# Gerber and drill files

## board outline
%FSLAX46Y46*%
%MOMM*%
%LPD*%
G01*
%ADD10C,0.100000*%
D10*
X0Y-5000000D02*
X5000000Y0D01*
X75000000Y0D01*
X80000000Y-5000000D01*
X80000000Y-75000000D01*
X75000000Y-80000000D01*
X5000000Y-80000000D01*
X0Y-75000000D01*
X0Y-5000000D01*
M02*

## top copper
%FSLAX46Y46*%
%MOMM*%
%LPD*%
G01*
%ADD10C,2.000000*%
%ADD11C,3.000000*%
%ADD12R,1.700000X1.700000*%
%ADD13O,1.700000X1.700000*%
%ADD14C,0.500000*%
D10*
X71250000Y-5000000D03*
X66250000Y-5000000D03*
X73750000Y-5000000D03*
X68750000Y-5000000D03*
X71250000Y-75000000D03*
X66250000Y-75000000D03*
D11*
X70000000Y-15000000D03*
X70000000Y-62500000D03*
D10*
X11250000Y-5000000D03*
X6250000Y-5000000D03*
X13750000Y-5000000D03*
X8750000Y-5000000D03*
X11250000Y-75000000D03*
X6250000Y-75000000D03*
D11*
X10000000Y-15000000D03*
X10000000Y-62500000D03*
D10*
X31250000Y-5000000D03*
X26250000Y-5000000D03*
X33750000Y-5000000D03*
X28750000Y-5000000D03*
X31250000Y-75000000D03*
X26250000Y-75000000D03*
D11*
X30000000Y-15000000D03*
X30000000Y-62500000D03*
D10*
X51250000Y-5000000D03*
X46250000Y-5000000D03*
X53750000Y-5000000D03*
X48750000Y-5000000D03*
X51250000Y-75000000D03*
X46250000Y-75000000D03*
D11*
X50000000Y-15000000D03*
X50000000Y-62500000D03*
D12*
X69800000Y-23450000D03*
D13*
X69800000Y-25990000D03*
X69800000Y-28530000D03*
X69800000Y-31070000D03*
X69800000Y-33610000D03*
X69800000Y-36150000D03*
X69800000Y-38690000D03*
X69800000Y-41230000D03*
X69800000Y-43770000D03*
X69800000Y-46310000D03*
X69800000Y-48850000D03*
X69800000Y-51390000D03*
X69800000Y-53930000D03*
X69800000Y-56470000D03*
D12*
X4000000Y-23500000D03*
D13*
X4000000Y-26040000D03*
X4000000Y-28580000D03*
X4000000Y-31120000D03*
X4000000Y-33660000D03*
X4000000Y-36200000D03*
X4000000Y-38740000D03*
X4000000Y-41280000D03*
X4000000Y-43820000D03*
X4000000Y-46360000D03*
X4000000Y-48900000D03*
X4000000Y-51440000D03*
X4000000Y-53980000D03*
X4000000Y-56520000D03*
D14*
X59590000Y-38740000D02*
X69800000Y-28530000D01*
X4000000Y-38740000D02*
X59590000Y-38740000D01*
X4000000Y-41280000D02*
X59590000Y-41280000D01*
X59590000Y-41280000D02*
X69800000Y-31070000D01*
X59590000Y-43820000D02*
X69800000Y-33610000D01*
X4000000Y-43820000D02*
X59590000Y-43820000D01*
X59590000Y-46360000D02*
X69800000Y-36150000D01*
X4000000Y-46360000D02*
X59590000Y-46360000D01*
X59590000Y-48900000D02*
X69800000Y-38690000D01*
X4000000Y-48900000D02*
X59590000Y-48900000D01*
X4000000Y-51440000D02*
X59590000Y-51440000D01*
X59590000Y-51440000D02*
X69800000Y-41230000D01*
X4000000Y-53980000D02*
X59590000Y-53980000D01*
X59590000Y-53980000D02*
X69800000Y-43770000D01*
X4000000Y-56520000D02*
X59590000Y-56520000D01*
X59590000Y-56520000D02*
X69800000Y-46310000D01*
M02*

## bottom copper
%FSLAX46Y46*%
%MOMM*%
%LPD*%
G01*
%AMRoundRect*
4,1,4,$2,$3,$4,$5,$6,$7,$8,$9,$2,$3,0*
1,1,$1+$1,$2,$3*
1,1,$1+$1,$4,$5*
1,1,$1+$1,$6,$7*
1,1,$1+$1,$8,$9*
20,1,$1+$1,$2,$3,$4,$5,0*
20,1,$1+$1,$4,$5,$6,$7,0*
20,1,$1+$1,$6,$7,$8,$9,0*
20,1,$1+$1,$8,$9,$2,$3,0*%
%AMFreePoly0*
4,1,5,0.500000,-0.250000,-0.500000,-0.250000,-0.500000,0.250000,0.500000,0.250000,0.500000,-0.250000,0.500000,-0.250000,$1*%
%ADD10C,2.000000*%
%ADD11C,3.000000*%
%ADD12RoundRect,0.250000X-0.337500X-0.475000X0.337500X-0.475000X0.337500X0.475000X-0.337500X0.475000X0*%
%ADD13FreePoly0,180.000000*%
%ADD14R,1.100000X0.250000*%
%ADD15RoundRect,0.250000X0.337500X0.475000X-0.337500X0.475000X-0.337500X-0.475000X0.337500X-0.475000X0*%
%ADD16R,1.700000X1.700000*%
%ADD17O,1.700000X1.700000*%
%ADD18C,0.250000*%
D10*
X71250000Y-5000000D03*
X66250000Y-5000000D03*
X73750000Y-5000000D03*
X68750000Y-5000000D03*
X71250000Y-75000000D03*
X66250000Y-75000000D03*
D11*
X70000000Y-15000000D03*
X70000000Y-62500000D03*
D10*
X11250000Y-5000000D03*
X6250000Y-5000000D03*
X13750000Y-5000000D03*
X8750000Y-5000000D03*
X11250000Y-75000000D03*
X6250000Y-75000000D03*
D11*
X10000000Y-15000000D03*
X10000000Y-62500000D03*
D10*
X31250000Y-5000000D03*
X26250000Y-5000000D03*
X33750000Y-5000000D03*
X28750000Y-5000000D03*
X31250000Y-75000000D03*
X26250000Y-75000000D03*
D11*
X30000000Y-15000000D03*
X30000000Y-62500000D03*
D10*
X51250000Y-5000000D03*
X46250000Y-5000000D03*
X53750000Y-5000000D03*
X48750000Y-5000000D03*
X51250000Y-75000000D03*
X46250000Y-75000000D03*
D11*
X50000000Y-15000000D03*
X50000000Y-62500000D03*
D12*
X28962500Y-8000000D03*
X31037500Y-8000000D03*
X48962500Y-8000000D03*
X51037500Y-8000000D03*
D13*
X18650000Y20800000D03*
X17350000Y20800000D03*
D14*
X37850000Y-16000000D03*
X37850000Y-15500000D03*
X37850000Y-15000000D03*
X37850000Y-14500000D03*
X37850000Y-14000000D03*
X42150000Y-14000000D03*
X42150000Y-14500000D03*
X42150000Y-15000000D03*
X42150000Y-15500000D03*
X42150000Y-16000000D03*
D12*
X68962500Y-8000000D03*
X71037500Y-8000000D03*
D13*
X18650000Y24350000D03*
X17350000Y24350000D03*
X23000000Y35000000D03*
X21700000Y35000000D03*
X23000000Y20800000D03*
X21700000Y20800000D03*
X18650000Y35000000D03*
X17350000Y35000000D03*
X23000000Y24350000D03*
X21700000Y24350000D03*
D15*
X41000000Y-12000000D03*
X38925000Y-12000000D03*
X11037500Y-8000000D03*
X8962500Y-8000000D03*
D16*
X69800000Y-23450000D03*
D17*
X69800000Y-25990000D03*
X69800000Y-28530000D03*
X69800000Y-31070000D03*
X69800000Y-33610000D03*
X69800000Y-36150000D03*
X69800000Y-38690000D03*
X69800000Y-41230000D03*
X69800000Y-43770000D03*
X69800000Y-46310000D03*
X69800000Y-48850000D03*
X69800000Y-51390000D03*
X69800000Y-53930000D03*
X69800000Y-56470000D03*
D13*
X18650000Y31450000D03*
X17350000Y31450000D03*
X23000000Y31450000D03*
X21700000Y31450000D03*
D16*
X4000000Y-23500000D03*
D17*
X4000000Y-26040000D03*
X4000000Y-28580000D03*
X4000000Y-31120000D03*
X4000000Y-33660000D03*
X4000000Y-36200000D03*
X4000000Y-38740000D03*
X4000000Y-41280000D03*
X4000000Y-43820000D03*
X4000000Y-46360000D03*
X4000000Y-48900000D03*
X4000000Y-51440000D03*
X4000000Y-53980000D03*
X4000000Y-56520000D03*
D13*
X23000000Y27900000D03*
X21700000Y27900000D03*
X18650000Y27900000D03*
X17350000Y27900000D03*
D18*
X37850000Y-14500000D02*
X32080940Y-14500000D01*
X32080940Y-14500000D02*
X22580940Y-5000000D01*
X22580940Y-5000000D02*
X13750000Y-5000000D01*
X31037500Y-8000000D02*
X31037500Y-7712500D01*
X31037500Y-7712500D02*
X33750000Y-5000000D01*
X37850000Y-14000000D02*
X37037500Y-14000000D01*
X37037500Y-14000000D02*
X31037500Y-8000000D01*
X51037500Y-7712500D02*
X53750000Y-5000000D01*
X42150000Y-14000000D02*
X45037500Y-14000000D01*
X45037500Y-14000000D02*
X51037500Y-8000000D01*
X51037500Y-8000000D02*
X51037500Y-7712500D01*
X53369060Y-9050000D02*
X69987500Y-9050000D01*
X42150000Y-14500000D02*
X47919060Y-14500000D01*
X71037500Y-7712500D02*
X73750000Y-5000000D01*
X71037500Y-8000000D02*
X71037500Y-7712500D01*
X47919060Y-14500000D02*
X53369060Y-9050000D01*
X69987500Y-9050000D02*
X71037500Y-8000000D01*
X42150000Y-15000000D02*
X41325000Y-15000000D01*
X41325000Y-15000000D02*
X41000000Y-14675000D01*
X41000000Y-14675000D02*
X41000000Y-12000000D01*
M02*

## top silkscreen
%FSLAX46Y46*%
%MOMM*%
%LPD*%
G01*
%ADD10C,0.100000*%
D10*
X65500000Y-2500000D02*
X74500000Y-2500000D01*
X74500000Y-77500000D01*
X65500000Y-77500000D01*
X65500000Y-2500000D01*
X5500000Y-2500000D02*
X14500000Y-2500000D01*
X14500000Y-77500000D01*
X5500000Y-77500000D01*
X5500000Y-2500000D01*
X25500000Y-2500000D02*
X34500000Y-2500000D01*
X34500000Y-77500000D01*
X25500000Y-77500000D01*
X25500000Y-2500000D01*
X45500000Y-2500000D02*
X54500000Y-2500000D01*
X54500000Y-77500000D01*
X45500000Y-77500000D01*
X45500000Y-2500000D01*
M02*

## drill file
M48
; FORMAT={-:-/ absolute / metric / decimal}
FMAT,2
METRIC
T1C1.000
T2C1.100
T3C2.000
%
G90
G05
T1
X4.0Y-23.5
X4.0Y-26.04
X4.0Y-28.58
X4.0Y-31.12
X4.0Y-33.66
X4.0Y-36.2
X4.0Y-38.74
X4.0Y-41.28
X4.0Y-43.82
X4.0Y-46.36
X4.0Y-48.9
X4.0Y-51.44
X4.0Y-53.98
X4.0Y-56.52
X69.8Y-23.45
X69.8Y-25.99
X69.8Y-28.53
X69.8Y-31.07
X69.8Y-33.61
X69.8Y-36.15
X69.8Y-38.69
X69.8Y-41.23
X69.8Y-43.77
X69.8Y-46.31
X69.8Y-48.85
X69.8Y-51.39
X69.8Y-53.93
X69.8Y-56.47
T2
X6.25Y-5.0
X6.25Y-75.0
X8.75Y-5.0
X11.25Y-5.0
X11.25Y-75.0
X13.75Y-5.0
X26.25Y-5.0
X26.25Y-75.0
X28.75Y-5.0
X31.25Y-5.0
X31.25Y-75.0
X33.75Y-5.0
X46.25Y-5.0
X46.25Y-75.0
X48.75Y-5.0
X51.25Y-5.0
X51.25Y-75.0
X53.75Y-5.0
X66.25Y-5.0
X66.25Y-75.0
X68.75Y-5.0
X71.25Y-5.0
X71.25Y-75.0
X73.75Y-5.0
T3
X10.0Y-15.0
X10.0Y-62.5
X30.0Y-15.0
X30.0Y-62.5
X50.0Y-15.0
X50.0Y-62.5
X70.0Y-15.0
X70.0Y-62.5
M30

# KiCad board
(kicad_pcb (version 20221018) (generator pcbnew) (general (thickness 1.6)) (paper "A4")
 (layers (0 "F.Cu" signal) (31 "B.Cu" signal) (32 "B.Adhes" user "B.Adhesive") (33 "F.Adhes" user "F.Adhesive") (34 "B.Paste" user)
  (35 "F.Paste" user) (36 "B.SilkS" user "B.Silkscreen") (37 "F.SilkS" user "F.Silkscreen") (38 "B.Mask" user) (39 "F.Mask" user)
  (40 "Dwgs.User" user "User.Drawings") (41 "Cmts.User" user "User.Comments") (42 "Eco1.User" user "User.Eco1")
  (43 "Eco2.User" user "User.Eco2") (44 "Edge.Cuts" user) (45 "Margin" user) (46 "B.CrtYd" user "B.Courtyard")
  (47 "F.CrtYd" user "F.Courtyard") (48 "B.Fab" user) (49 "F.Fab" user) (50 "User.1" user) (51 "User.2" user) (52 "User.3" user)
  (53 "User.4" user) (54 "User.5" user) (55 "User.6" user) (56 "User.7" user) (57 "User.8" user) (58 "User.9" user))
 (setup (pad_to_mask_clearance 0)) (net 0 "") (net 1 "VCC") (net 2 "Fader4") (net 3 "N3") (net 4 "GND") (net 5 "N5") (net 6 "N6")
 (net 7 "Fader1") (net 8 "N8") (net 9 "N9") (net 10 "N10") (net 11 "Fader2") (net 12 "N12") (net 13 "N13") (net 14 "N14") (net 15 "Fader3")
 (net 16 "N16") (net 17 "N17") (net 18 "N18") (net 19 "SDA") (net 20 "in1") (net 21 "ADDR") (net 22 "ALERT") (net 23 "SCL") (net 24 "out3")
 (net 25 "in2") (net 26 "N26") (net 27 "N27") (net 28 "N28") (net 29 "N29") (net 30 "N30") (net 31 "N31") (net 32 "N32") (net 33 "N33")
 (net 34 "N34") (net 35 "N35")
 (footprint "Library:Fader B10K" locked (layer "F.Cu") (at 70 5 -90)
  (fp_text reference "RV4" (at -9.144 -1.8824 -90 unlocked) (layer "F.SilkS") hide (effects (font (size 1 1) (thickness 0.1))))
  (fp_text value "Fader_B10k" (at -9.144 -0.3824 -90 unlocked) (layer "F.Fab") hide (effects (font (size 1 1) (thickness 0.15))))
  (fp_rect (start -2.5 -4.5) (end 72.5 4.5) (stroke (width 0.1) (type default)) (fill none) (layer "F.SilkS"))
  (pad "1" thru_hole circle locked (at 0 -1.25 270) (size 2 2) (drill 1.1) (layers "*.Cu" "*.Mask") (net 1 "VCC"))
  (pad "1'" thru_hole circle locked (at 0 3.75 270) (size 2 2) (drill 1.1) (layers "*.Cu" "*.Mask") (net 1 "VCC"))
  (pad "2" thru_hole circle locked (at 0 -3.75 270) (size 2 2) (drill 1.1) (layers "*.Cu" "*.Mask") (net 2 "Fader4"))
  (pad "2'" thru_hole circle locked (at 0 1.25 270) (size 2 2) (drill 1.1) (layers "*.Cu" "*.Mask") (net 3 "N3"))
  (pad "3" thru_hole circle locked (at 70 -1.25 270) (size 2 2) (drill 1.1) (layers "*.Cu" "*.Mask") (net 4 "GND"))
  (pad "3'" thru_hole circle locked (at 70 3.75 270) (size 2 2) (drill 1.1) (layers "*.Cu" "*.Mask") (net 4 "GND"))
  (pad "4" thru_hole circle locked (at 10 0 270) (size 3 3) (drill 2) (layers "*.Cu" "*.Mask") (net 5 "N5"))
  (pad "5" thru_hole circle locked (at 57.5 0 270) (size 3 3) (drill 2) (layers "*.Cu" "*.Mask") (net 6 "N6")))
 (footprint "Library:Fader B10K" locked (layer "F.Cu") (at 10 5 -90)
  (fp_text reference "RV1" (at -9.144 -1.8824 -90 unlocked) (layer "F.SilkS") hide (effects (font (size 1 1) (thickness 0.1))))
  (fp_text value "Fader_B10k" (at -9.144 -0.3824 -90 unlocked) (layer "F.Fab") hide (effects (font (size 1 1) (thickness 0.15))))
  (fp_rect (start -2.5 -4.5) (end 72.5 4.5) (stroke (width 0.1) (type default)) (fill none) (layer "F.SilkS"))
  (pad "1" thru_hole circle locked (at 0 -1.25 270) (size 2 2) (drill 1.1) (layers "*.Cu" "*.Mask") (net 1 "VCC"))
  (pad "1'" thru_hole circle locked (at 0 3.75 270) (size 2 2) (drill 1.1) (layers "*.Cu" "*.Mask") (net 1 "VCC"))
  (pad "2" thru_hole circle locked (at 0 -3.75 270) (size 2 2) (drill 1.1) (layers "*.Cu" "*.Mask") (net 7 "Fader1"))
  (pad "2'" thru_hole circle locked (at 0 1.25 270) (size 2 2) (drill 1.1) (layers "*.Cu" "*.Mask") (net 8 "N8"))
  (pad "3" thru_hole circle locked (at 70 -1.25 270) (size 2 2) (drill 1.1) (layers "*.Cu" "*.Mask") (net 4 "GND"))
  (pad "3'" thru_hole circle locked (at 70 3.75 270) (size 2 2) (drill 1.1) (layers "*.Cu" "*.Mask") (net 4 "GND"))
  (pad "4" thru_hole circle locked (at 10 0 270) (size 3 3) (drill 2) (layers "*.Cu" "*.Mask") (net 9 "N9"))
  (pad "5" thru_hole circle locked (at 57.5 0 270) (size 3 3) (drill 2) (layers "*.Cu" "*.Mask") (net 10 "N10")))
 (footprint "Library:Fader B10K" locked (layer "F.Cu") (at 30 5 -90)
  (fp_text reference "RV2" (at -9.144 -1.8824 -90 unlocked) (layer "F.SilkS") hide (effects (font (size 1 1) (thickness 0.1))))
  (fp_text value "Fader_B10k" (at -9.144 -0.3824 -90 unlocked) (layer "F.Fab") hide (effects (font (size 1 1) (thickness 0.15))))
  (fp_rect (start -2.5 -4.5) (end 72.5 4.5) (stroke (width 0.1) (type default)) (fill none) (layer "F.SilkS"))
  (pad "1" thru_hole circle locked (at 0 -1.25 270) (size 2 2) (drill 1.1) (layers "*.Cu" "*.Mask") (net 1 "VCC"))
  (pad "1'" thru_hole circle locked (at 0 3.75 270) (size 2 2) (drill 1.1) (layers "*.Cu" "*.Mask") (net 1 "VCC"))
  (pad "2" thru_hole circle locked (at 0 -3.75 270) (size 2 2) (drill 1.1) (layers "*.Cu" "*.Mask") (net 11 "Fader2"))
  (pad "2'" thru_hole circle locked (at 0 1.25 270) (size 2 2) (drill 1.1) (layers "*.Cu" "*.Mask") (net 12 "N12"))
  (pad "3" thru_hole circle locked (at 70 -1.25 270) (size 2 2) (drill 1.1) (layers "*.Cu" "*.Mask") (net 4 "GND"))
  (pad "3'" thru_hole circle locked (at 70 3.75 270) (size 2 2) (drill 1.1) (layers "*.Cu" "*.Mask") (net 4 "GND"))
  (pad "4" thru_hole circle locked (at 10 0 270) (size 3 3) (drill 2) (layers "*.Cu" "*.Mask") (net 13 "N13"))
  (pad "5" thru_hole circle locked (at 57.5 0 270) (size 3 3) (drill 2) (layers "*.Cu" "*.Mask") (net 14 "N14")))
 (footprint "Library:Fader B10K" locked (layer "F.Cu") (at 50 5 -90)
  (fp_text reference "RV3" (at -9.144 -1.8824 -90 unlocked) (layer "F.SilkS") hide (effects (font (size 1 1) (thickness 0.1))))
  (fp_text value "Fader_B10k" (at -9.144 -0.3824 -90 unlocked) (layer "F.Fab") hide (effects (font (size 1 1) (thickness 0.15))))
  (fp_rect (start -2.5 -4.5) (end 72.5 4.5) (stroke (width 0.1) (type default)) (fill none) (layer "F.SilkS"))
  (pad "1" thru_hole circle locked (at 0 -1.25 270) (size 2 2) (drill 1.1) (layers "*.Cu" "*.Mask") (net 1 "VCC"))
  (pad "1'" thru_hole circle locked (at 0 3.75 270) (size 2 2) (drill 1.1) (layers "*.Cu" "*.Mask") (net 1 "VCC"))
  (pad "2" thru_hole circle locked (at 0 -3.75 270) (size 2 2) (drill 1.1) (layers "*.Cu" "*.Mask") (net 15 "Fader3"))
  (pad "2'" thru_hole circle locked (at 0 1.25 270) (size 2 2) (drill 1.1) (layers "*.Cu" "*.Mask") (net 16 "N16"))
  (pad "3" thru_hole circle locked (at 70 -1.25 270) (size 2 2) (drill 1.1) (layers "*.Cu" "*.Mask") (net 4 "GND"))
  (pad "3'" thru_hole circle locked (at 70 3.75 270) (size 2 2) (drill 1.1) (layers "*.Cu" "*.Mask") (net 4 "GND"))
  (pad "4" thru_hole circle locked (at 10 0 270) (size 3 3) (drill 2) (layers "*.Cu" "*.Mask") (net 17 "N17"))
  (pad "5" thru_hole circle locked (at 57.5 0 270) (size 3 3) (drill 2) (layers "*.Cu" "*.Mask") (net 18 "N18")))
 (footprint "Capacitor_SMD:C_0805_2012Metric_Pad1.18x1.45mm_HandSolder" (layer "B.Cu") (at 30 8)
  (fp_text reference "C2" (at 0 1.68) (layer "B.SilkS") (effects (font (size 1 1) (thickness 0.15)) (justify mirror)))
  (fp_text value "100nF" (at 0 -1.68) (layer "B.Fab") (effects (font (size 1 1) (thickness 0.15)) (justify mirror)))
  (pad "1" smd roundrect (at -1.0375 0) (size 1.175 1.45) (layers "B.Cu" "B.Paste" "B.Mask") (roundrect_rratio 0.212766) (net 4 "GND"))
  (pad "2" smd roundrect (at 1.0375 0) (size 1.175 1.45) (layers "B.Cu" "B.Paste" "B.Mask") (roundrect_rratio 0.212766) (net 11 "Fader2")))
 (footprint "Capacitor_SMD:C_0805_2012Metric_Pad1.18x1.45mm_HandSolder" (layer "B.Cu") (at 50 8)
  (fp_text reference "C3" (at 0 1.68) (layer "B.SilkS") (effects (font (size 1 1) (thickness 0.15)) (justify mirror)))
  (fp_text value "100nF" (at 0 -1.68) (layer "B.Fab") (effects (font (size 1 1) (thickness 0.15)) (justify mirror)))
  (pad "1" smd roundrect (at -1.0375 0) (size 1.175 1.45) (layers "B.Cu" "B.Paste" "B.Mask") (roundrect_rratio 0.212766) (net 4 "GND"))
  (pad "2" smd roundrect (at 1.0375 0) (size 1.175 1.45) (layers "B.Cu" "B.Paste" "B.Mask") (roundrect_rratio 0.212766) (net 15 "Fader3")))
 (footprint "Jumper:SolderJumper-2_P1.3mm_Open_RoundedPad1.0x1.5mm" (layer "B.Cu") (at 18 -20.8 180)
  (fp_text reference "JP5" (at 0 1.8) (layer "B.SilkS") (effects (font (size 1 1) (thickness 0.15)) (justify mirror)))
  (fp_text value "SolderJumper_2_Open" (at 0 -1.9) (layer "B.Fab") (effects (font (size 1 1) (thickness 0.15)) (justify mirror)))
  (pad "1" smd custom (at -0.65 0 180) (size 1 0.5) (layers "B.Cu" "B.Mask") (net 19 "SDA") (zone_connect 2)
   (options (clearance outline) (anchor rect)) (primitives))
  (pad "2" smd custom (at 0.65 0 180) (size 1 0.5) (layers "B.Cu" "B.Mask") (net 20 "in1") (zone_connect 2)
   (options (clearance outline) (anchor rect)) (primitives)))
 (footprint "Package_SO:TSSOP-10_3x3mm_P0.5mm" (layer "B.Cu") (at 40 15)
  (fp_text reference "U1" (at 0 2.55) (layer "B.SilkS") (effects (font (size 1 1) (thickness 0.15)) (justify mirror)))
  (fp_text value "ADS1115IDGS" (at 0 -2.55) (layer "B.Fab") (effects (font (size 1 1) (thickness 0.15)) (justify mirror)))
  (pad "1" smd rect (at -2.15 1) (size 1.1 0.25) (layers "B.Cu" "B.Paste" "B.Mask") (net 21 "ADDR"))
  (pad "2" smd rect (at -2.15 0.5) (size 1.1 0.25) (layers "B.Cu" "B.Paste" "B.Mask") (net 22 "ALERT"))
  (pad "3" smd rect (at -2.15 0) (size 1.1 0.25) (layers "B.Cu" "B.Paste" "B.Mask") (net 4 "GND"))
  (pad "4" smd rect (at -2.15 -0.5) (size 1.1 0.25) (layers "B.Cu" "B.Paste" "B.Mask") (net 7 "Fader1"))
  (pad "5" smd rect (at -2.15 -1) (size 1.1 0.25) (layers "B.Cu" "B.Paste" "B.Mask") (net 11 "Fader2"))
  (pad "6" smd rect (at 2.15 -1) (size 1.1 0.25) (layers "B.Cu" "B.Paste" "B.Mask") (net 15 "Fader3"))
  (pad "7" smd rect (at 2.15 -0.5) (size 1.1 0.25) (layers "B.Cu" "B.Paste" "B.Mask") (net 2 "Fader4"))
  (pad "8" smd rect (at 2.15 0) (size 1.1 0.25) (layers "B.Cu" "B.Paste" "B.Mask") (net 1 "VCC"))
  (pad "9" smd rect (at 2.15 0.5) (size 1.1 0.25) (layers "B.Cu" "B.Paste" "B.Mask") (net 19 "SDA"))
  (pad "10" smd rect (at 2.15 1) (size 1.1 0.25) (layers "B.Cu" "B.Paste" "B.Mask") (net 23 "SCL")))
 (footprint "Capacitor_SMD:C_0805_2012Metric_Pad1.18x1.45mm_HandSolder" (layer "B.Cu") (at 70 8)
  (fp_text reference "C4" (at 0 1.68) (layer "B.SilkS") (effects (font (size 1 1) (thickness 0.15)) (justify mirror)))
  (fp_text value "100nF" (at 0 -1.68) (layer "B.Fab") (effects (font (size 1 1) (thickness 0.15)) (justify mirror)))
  (pad "1" smd roundrect (at -1.0375 0) (size 1.175 1.45) (layers "B.Cu" "B.Paste" "B.Mask") (roundrect_rratio 0.212766) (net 4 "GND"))
  (pad "2" smd roundrect (at 1.0375 0) (size 1.175 1.45) (layers "B.Cu" "B.Paste" "B.Mask") (roundrect_rratio 0.212766) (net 2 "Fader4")))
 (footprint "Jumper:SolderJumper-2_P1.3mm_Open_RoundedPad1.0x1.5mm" (layer "B.Cu") (at 18 -24.35 180)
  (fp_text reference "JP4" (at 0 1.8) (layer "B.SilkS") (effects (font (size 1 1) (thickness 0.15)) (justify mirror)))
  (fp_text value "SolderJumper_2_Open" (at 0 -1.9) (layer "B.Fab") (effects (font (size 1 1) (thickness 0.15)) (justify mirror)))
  (pad "1" smd custom (at -0.65 0 180) (size 1 0.5) (layers "B.Cu" "B.Mask") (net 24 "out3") (zone_connect 2)
   (options (clearance outline) (anchor rect)) (primitives))
  (pad "2" smd custom (at 0.65 0 180) (size 1 0.5) (layers "B.Cu" "B.Mask") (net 2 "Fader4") (zone_connect 2)
   (options (clearance outline) (anchor rect)) (primitives)))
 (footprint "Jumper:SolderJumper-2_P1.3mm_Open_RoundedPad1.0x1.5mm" (layer "B.Cu") (at 22.35 -35 180)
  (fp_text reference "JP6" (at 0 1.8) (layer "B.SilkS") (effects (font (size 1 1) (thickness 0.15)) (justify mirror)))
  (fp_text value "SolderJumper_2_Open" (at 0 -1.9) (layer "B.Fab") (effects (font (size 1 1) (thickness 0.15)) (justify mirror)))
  (pad "1" smd custom (at -0.65 0 180) (size 1 0.5) (layers "B.Cu" "B.Mask") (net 23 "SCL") (zone_connect 2)
   (options (clearance outline) (anchor rect)) (primitives))
  (pad "2" smd custom (at 0.65 0 180) (size 1 0.5) (layers "B.Cu" "B.Mask") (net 20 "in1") (zone_connect 2)
   (options (clearance outline) (anchor rect)) (primitives)))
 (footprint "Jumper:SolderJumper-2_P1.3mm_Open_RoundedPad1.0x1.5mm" (layer "B.Cu") (at 22.35 -20.8 180)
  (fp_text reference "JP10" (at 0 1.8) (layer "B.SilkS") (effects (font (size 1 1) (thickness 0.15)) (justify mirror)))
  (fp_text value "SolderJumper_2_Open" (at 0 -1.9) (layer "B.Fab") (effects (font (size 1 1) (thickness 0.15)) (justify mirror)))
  (pad "1" smd custom (at -0.65 0 180) (size 1 0.5) (layers "B.Cu" "B.Mask") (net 21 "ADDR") (zone_connect 2)
   (options (clearance outline) (anchor rect)) (primitives))
  (pad "2" smd custom (at 0.65 0 180) (size 1 0.5) (layers "B.Cu" "B.Mask") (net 23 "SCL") (zone_connect 2)
   (options (clearance outline) (anchor rect)) (primitives)))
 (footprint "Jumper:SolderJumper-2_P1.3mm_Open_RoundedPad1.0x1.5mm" (layer "B.Cu") (at 18 -35 180)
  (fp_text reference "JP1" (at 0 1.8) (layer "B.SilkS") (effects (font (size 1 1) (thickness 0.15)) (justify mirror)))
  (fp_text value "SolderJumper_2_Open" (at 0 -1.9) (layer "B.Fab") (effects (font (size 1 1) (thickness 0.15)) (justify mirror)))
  (pad "1" smd custom (at -0.65 0 180) (size 1 0.5) (layers "B.Cu" "B.Mask") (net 19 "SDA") (zone_connect 2)
   (options (clearance outline) (anchor rect)) (primitives))
  (pad "2" smd custom (at 0.65 0 180) (size 1 0.5) (layers "B.Cu" "B.Mask") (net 7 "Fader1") (zone_connect 2)
   (options (clearance outline) (anchor rect)) (primitives)))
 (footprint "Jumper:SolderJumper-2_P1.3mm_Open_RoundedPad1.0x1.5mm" (layer "B.Cu") (at 22.35 -24.35 180)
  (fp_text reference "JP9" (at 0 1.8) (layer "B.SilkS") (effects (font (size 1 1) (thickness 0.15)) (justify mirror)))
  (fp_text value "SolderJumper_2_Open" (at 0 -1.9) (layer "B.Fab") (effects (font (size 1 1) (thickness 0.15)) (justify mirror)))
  (pad "1" smd custom (at -0.65 0 180) (size 1 0.5) (layers "B.Cu" "B.Mask") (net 21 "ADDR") (zone_connect 2)
   (options (clearance outline) (anchor rect)) (primitives))
  (pad "2" smd custom (at 0.65 0 180) (size 1 0.5) (layers "B.Cu" "B.Mask") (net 19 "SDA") (zone_connect 2)
   (options (clearance outline) (anchor rect)) (primitives)))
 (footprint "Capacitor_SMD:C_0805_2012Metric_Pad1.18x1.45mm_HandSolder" (layer "B.Cu") (at 39.9625 12 180)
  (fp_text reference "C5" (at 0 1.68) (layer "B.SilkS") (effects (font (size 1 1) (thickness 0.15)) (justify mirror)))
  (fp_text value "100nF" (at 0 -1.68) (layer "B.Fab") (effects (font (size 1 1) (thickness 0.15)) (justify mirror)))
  (pad "1" smd roundrect (at -1.0375 0 180) (size 1.175 1.45) (layers "B.Cu" "B.Paste" "B.Mask") (roundrect_rratio 0.212766) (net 1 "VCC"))
  (pad "2" smd roundrect (at 1.0375 0 180) (size 1.175 1.45) (layers "B.Cu" "B.Paste" "B.Mask") (roundrect_rratio 0.212766) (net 4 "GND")))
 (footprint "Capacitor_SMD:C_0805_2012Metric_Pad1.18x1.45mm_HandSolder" (layer "B.Cu") (at 10 8 180)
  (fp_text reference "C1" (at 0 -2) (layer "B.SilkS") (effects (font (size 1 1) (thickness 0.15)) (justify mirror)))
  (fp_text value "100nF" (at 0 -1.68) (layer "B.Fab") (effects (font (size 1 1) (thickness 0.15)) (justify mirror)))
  (pad "1" smd roundrect (at -1.0375 0 180) (size 1.175 1.45) (layers "B.Cu" "B.Paste" "B.Mask") (roundrect_rratio 0.212766) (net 4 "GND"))
  (pad "2" smd roundrect (at 1.0375 0 180) (size 1.175 1.45) (layers "B.Cu" "B.Paste" "B.Mask") (roundrect_rratio 0.212766) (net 7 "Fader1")))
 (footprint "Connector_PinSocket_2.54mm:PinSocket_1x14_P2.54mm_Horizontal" (layer "B.Cu") (at 69.8 23.45 180)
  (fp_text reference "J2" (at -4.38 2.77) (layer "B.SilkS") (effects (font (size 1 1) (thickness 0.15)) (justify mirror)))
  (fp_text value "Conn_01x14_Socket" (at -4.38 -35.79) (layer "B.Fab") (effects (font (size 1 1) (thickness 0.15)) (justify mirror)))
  (pad "1" thru_hole rect (at 0 0 180) (size 1.7 1.7) (drill 1) (layers "*.Cu" "*.Mask") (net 1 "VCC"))
  (pad "2" thru_hole oval (at 0 -2.54 180) (size 1.7 1.7) (drill 1) (layers "*.Cu" "*.Mask") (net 4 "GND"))
  (pad "3" thru_hole oval (at 0 -5.08 180) (size 1.7 1.7) (drill 1) (layers "*.Cu" "*.Mask") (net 20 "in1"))
  (pad "4" thru_hole oval (at 0 -7.62 180) (size 1.7 1.7) (drill 1) (layers "*.Cu" "*.Mask") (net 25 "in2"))
  (pad "5" thru_hole oval (at 0 -10.16 180) (size 1.7 1.7) (drill 1) (layers "*.Cu" "*.Mask") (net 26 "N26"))
  (pad "6" thru_hole oval (at 0 -12.7 180) (size 1.7 1.7) (drill 1) (layers "*.Cu" "*.Mask") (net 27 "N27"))
  (pad "7" thru_hole oval (at 0 -15.24 180) (size 1.7 1.7) (drill 1) (layers "*.Cu" "*.Mask") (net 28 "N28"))
  (pad "8" thru_hole oval (at 0 -17.78 180) (size 1.7 1.7) (drill 1) (layers "*.Cu" "*.Mask") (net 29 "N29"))
  (pad "9" thru_hole oval (at 0 -20.32 180) (size 1.7 1.7) (drill 1) (layers "*.Cu" "*.Mask") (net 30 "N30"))
  (pad "10" thru_hole oval (at 0 -22.86 180) (size 1.7 1.7) (drill 1) (layers "*.Cu" "*.Mask") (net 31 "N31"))
  (pad "11" thru_hole oval (at 0 -25.4 180) (size 1.7 1.7) (drill 1) (layers "*.Cu" "*.Mask") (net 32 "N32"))
  (pad "12" thru_hole oval (at 0 -27.94 180) (size 1.7 1.7) (drill 1) (layers "*.Cu" "*.Mask") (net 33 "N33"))
  (pad "13" thru_hole oval (at 0 -30.48 180) (size 1.7 1.7) (drill 1) (layers "*.Cu" "*.Mask") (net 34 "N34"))
  (pad "14" thru_hole oval (at 0 -33.02 180) (size 1.7 1.7) (drill 1) (layers "*.Cu" "*.Mask") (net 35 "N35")))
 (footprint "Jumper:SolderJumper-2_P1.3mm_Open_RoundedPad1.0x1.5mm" (layer "B.Cu") (at 18 -31.45 180)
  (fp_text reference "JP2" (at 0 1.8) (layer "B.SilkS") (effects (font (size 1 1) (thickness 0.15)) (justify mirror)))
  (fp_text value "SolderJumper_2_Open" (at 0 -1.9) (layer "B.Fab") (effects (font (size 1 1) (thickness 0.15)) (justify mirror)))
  (pad "1" smd custom (at -0.65 0 180) (size 1 0.5) (layers "B.Cu" "B.Mask") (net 23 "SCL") (zone_connect 2)
   (options (clearance outline) (anchor rect)) (primitives))
  (pad "2" smd custom (at 0.65 0 180) (size 1 0.5) (layers "B.Cu" "B.Mask") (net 11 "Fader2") (zone_connect 2)
   (options (clearance outline) (anchor rect)) (primitives)))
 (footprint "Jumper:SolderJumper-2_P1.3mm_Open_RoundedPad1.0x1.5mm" (layer "B.Cu") (at 22.35 -31.45 180)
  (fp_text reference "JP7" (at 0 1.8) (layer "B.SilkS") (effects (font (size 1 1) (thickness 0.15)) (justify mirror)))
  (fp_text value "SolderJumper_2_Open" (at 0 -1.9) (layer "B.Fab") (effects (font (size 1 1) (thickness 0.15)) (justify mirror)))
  (pad "1" smd custom (at -0.65 0 180) (size 1 0.5) (layers "B.Cu" "B.Mask") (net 21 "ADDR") (zone_connect 2)
   (options (clearance outline) (anchor rect)) (primitives))
  (pad "2" smd custom (at 0.65 0 180) (size 1 0.5) (layers "B.Cu" "B.Mask") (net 4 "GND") (zone_connect 2)
   (options (clearance outline) (anchor rect)) (primitives)))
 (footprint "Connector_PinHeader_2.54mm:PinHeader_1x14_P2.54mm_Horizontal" (layer "B.Cu") (at 4 23.5 180)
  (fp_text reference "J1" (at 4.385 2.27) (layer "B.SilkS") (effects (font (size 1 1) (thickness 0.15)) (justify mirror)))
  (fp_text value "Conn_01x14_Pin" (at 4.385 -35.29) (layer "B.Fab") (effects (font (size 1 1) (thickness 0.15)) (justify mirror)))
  (pad "1" thru_hole rect (at 0 0 180) (size 1.7 1.7) (drill 1) (layers "*.Cu" "*.Mask") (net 1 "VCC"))
  (pad "2" thru_hole oval (at 0 -2.54 180) (size 1.7 1.7) (drill 1) (layers "*.Cu" "*.Mask") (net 4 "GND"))
  (pad "3" thru_hole oval (at 0 -5.08 180) (size 1.7 1.7) (drill 1) (layers "*.Cu" "*.Mask") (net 19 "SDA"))
  (pad "4" thru_hole oval (at 0 -7.62 180) (size 1.7 1.7) (drill 1) (layers "*.Cu" "*.Mask") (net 23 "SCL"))
  (pad "5" thru_hole oval (at 0 -10.16 180) (size 1.7 1.7) (drill 1) (layers "*.Cu" "*.Mask") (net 24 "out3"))
  (pad "6" thru_hole oval (at 0 -12.7 180) (size 1.7 1.7) (drill 1) (layers "*.Cu" "*.Mask") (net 24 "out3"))
  (pad "7" thru_hole oval (at 0 -15.24 180) (size 1.7 1.7) (drill 1) (layers "*.Cu" "*.Mask") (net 20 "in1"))
  (pad "8" thru_hole oval (at 0 -17.78 180) (size 1.7 1.7) (drill 1) (layers "*.Cu" "*.Mask") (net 25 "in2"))
  (pad "9" thru_hole oval (at 0 -20.32 180) (size 1.7 1.7) (drill 1) (layers "*.Cu" "*.Mask") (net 26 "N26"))
  (pad "10" thru_hole oval (at 0 -22.86 180) (size 1.7 1.7) (drill 1) (layers "*.Cu" "*.Mask") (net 27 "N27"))
  (pad "11" thru_hole oval (at 0 -25.4 180) (size 1.7 1.7) (drill 1) (layers "*.Cu" "*.Mask") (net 28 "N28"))
  (pad "12" thru_hole oval (at 0 -27.94 180) (size 1.7 1.7) (drill 1) (layers "*.Cu" "*.Mask") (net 29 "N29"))
  (pad "13" thru_hole oval (at 0 -30.48 180) (size 1.7 1.7) (drill 1) (layers "*.Cu" "*.Mask") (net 30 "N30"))
  (pad "14" thru_hole oval (at 0 -33.02 180) (size 1.7 1.7) (drill 1) (layers "*.Cu" "*.Mask") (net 31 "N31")))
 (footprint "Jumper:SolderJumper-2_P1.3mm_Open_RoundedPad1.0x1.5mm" (layer "B.Cu") (at 22.35 -27.9 180)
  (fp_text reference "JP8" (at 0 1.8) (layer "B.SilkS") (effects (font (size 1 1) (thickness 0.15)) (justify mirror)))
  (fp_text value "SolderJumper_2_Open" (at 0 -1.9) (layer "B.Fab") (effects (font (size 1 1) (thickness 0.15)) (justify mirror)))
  (pad "1" smd custom (at -0.65 0 180) (size 1 0.5) (layers "B.Cu" "B.Mask") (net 21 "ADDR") (zone_connect 2)
   (options (clearance outline) (anchor rect)) (primitives))
  (pad "2" smd custom (at 0.65 0 180) (size 1 0.5) (layers "B.Cu" "B.Mask") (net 1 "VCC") (zone_connect 2)
   (options (clearance outline) (anchor rect)) (primitives)))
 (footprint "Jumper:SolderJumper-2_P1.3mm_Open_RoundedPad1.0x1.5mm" (layer "B.Cu") (at 18 -27.9 180)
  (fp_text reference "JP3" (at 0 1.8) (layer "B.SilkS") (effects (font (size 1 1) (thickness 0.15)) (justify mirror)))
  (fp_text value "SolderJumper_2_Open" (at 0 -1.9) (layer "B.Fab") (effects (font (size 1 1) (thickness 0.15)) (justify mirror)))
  (pad "1" smd custom (at -0.65 0 180) (size 1 0.5) (layers "B.Cu" "B.Mask") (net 24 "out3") (zone_connect 2)
   (options (clearance outline) (anchor rect)) (primitives))
  (pad "2" smd custom (at 0.65 0 180) (size 1 0.5) (layers "B.Cu" "B.Mask") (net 15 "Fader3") (zone_connect 2)
   (options (clearance outline) (anchor rect)) (primitives)))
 (gr_poly
  (pts (xy 0 5) (xy 5 0) (xy 75 0) (xy 80 5) (xy 80 75) (xy 75 80) (xy 5 80) (xy 0 75)) (stroke (width 0.1) (type solid)) (fill none)
  (layer "Edge.Cuts"))
 (segment (start 37.85 14.5) (end 32.08094 14.5) (width 0.25) (layer "B.Cu") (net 7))
 (segment (start 32.08094 14.5) (end 22.58094 5) (width 0.25) (layer "B.Cu") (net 7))
 (segment (start 22.58094 5) (end 13.75 5) (width 0.25) (layer "B.Cu") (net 7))
 (segment (start 31.0375 8) (end 31.0375 7.7125) (width 0.25) (layer "B.Cu") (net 11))
 (segment (start 31.0375 7.7125) (end 33.75 5) (width 0.25) (layer "B.Cu") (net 11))
 (segment (start 37.85 14) (end 37.0375 14) (width 0.25) (layer "B.Cu") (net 11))
 (segment (start 37.0375 14) (end 31.0375 8) (width 0.25) (layer "B.Cu") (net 11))
 (segment (start 51.0375 7.7125) (end 53.75 5) (width 0.25) (layer "B.Cu") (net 15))
 (segment (start 42.15 14) (end 45.0375 14) (width 0.25) (layer "B.Cu") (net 15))
 (segment (start 45.0375 14) (end 51.0375 8) (width 0.25) (layer "B.Cu") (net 15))
 (segment (start 51.0375 8) (end 51.0375 7.7125) (width 0.25) (layer "B.Cu") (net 15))
 (segment (start 53.36906 9.05) (end 69.9875 9.05) (width 0.25) (layer "B.Cu") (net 2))
 (segment (start 42.15 14.5) (end 47.91906 14.5) (width 0.25) (layer "B.Cu") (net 2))
 (segment (start 71.0375 7.7125) (end 73.75 5) (width 0.25) (layer "B.Cu") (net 2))
 (segment (start 71.0375 8) (end 71.0375 7.7125) (width 0.25) (layer "B.Cu") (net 2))
 (segment (start 47.91906 14.5) (end 53.36906 9.05) (width 0.25) (layer "B.Cu") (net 2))
 (segment (start 69.9875 9.05) (end 71.0375 8) (width 0.25) (layer "B.Cu") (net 2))
 (segment (start 42.15 15) (end 41.325 15) (width 0.25) (layer "B.Cu") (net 1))
 (segment (start 41.325 15) (end 41 14.675) (width 0.25) (layer "B.Cu") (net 1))
 (segment (start 41 14.675) (end 41 12) (width 0.25) (layer "B.Cu") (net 1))
 (segment (start 59.59 38.74) (end 69.8 28.53) (width 0.5) (layer "F.Cu") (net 20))
 (segment (start 4 38.74) (end 59.59 38.74) (width 0.5) (layer "F.Cu") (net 20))
 (segment (start 4 41.28) (end 59.59 41.28) (width 0.5) (layer "F.Cu") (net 25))
 (segment (start 59.59 41.28) (end 69.8 31.07) (width 0.5) (layer "F.Cu") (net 25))
 (segment (start 59.59 43.82) (end 69.8 33.61) (width 0.5) (layer "F.Cu") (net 26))
 (segment (start 4 43.82) (end 59.59 43.82) (width 0.5) (layer "F.Cu") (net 26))
 (segment (start 59.59 46.36) (end 69.8 36.15) (width 0.5) (layer "F.Cu") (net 27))
 (segment (start 4 46.36) (end 59.59 46.36) (width 0.5) (layer "F.Cu") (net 27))
 (segment (start 59.59 48.9) (end 69.8 38.69) (width 0.5) (layer "F.Cu") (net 28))
 (segment (start 4 48.9) (end 59.59 48.9) (width 0.5) (layer "F.Cu") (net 28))
 (segment (start 4 51.44) (end 59.59 51.44) (width 0.5) (layer "F.Cu") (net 29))
 (segment (start 59.59 51.44) (end 69.8 41.23) (width 0.5) (layer "F.Cu") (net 29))
 (segment (start 4 53.98) (end 59.59 53.98) (width 0.5) (layer "F.Cu") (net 30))
 (segment (start 59.59 53.98) (end 69.8 43.77) (width 0.5) (layer "F.Cu") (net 30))
 (segment (start 4 56.52) (end 59.59 56.52) (width 0.5) (layer "F.Cu") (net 31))
 (segment (start 59.59 56.52) (end 69.8 46.31) (width 0.5) (layer "F.Cu") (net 31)))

